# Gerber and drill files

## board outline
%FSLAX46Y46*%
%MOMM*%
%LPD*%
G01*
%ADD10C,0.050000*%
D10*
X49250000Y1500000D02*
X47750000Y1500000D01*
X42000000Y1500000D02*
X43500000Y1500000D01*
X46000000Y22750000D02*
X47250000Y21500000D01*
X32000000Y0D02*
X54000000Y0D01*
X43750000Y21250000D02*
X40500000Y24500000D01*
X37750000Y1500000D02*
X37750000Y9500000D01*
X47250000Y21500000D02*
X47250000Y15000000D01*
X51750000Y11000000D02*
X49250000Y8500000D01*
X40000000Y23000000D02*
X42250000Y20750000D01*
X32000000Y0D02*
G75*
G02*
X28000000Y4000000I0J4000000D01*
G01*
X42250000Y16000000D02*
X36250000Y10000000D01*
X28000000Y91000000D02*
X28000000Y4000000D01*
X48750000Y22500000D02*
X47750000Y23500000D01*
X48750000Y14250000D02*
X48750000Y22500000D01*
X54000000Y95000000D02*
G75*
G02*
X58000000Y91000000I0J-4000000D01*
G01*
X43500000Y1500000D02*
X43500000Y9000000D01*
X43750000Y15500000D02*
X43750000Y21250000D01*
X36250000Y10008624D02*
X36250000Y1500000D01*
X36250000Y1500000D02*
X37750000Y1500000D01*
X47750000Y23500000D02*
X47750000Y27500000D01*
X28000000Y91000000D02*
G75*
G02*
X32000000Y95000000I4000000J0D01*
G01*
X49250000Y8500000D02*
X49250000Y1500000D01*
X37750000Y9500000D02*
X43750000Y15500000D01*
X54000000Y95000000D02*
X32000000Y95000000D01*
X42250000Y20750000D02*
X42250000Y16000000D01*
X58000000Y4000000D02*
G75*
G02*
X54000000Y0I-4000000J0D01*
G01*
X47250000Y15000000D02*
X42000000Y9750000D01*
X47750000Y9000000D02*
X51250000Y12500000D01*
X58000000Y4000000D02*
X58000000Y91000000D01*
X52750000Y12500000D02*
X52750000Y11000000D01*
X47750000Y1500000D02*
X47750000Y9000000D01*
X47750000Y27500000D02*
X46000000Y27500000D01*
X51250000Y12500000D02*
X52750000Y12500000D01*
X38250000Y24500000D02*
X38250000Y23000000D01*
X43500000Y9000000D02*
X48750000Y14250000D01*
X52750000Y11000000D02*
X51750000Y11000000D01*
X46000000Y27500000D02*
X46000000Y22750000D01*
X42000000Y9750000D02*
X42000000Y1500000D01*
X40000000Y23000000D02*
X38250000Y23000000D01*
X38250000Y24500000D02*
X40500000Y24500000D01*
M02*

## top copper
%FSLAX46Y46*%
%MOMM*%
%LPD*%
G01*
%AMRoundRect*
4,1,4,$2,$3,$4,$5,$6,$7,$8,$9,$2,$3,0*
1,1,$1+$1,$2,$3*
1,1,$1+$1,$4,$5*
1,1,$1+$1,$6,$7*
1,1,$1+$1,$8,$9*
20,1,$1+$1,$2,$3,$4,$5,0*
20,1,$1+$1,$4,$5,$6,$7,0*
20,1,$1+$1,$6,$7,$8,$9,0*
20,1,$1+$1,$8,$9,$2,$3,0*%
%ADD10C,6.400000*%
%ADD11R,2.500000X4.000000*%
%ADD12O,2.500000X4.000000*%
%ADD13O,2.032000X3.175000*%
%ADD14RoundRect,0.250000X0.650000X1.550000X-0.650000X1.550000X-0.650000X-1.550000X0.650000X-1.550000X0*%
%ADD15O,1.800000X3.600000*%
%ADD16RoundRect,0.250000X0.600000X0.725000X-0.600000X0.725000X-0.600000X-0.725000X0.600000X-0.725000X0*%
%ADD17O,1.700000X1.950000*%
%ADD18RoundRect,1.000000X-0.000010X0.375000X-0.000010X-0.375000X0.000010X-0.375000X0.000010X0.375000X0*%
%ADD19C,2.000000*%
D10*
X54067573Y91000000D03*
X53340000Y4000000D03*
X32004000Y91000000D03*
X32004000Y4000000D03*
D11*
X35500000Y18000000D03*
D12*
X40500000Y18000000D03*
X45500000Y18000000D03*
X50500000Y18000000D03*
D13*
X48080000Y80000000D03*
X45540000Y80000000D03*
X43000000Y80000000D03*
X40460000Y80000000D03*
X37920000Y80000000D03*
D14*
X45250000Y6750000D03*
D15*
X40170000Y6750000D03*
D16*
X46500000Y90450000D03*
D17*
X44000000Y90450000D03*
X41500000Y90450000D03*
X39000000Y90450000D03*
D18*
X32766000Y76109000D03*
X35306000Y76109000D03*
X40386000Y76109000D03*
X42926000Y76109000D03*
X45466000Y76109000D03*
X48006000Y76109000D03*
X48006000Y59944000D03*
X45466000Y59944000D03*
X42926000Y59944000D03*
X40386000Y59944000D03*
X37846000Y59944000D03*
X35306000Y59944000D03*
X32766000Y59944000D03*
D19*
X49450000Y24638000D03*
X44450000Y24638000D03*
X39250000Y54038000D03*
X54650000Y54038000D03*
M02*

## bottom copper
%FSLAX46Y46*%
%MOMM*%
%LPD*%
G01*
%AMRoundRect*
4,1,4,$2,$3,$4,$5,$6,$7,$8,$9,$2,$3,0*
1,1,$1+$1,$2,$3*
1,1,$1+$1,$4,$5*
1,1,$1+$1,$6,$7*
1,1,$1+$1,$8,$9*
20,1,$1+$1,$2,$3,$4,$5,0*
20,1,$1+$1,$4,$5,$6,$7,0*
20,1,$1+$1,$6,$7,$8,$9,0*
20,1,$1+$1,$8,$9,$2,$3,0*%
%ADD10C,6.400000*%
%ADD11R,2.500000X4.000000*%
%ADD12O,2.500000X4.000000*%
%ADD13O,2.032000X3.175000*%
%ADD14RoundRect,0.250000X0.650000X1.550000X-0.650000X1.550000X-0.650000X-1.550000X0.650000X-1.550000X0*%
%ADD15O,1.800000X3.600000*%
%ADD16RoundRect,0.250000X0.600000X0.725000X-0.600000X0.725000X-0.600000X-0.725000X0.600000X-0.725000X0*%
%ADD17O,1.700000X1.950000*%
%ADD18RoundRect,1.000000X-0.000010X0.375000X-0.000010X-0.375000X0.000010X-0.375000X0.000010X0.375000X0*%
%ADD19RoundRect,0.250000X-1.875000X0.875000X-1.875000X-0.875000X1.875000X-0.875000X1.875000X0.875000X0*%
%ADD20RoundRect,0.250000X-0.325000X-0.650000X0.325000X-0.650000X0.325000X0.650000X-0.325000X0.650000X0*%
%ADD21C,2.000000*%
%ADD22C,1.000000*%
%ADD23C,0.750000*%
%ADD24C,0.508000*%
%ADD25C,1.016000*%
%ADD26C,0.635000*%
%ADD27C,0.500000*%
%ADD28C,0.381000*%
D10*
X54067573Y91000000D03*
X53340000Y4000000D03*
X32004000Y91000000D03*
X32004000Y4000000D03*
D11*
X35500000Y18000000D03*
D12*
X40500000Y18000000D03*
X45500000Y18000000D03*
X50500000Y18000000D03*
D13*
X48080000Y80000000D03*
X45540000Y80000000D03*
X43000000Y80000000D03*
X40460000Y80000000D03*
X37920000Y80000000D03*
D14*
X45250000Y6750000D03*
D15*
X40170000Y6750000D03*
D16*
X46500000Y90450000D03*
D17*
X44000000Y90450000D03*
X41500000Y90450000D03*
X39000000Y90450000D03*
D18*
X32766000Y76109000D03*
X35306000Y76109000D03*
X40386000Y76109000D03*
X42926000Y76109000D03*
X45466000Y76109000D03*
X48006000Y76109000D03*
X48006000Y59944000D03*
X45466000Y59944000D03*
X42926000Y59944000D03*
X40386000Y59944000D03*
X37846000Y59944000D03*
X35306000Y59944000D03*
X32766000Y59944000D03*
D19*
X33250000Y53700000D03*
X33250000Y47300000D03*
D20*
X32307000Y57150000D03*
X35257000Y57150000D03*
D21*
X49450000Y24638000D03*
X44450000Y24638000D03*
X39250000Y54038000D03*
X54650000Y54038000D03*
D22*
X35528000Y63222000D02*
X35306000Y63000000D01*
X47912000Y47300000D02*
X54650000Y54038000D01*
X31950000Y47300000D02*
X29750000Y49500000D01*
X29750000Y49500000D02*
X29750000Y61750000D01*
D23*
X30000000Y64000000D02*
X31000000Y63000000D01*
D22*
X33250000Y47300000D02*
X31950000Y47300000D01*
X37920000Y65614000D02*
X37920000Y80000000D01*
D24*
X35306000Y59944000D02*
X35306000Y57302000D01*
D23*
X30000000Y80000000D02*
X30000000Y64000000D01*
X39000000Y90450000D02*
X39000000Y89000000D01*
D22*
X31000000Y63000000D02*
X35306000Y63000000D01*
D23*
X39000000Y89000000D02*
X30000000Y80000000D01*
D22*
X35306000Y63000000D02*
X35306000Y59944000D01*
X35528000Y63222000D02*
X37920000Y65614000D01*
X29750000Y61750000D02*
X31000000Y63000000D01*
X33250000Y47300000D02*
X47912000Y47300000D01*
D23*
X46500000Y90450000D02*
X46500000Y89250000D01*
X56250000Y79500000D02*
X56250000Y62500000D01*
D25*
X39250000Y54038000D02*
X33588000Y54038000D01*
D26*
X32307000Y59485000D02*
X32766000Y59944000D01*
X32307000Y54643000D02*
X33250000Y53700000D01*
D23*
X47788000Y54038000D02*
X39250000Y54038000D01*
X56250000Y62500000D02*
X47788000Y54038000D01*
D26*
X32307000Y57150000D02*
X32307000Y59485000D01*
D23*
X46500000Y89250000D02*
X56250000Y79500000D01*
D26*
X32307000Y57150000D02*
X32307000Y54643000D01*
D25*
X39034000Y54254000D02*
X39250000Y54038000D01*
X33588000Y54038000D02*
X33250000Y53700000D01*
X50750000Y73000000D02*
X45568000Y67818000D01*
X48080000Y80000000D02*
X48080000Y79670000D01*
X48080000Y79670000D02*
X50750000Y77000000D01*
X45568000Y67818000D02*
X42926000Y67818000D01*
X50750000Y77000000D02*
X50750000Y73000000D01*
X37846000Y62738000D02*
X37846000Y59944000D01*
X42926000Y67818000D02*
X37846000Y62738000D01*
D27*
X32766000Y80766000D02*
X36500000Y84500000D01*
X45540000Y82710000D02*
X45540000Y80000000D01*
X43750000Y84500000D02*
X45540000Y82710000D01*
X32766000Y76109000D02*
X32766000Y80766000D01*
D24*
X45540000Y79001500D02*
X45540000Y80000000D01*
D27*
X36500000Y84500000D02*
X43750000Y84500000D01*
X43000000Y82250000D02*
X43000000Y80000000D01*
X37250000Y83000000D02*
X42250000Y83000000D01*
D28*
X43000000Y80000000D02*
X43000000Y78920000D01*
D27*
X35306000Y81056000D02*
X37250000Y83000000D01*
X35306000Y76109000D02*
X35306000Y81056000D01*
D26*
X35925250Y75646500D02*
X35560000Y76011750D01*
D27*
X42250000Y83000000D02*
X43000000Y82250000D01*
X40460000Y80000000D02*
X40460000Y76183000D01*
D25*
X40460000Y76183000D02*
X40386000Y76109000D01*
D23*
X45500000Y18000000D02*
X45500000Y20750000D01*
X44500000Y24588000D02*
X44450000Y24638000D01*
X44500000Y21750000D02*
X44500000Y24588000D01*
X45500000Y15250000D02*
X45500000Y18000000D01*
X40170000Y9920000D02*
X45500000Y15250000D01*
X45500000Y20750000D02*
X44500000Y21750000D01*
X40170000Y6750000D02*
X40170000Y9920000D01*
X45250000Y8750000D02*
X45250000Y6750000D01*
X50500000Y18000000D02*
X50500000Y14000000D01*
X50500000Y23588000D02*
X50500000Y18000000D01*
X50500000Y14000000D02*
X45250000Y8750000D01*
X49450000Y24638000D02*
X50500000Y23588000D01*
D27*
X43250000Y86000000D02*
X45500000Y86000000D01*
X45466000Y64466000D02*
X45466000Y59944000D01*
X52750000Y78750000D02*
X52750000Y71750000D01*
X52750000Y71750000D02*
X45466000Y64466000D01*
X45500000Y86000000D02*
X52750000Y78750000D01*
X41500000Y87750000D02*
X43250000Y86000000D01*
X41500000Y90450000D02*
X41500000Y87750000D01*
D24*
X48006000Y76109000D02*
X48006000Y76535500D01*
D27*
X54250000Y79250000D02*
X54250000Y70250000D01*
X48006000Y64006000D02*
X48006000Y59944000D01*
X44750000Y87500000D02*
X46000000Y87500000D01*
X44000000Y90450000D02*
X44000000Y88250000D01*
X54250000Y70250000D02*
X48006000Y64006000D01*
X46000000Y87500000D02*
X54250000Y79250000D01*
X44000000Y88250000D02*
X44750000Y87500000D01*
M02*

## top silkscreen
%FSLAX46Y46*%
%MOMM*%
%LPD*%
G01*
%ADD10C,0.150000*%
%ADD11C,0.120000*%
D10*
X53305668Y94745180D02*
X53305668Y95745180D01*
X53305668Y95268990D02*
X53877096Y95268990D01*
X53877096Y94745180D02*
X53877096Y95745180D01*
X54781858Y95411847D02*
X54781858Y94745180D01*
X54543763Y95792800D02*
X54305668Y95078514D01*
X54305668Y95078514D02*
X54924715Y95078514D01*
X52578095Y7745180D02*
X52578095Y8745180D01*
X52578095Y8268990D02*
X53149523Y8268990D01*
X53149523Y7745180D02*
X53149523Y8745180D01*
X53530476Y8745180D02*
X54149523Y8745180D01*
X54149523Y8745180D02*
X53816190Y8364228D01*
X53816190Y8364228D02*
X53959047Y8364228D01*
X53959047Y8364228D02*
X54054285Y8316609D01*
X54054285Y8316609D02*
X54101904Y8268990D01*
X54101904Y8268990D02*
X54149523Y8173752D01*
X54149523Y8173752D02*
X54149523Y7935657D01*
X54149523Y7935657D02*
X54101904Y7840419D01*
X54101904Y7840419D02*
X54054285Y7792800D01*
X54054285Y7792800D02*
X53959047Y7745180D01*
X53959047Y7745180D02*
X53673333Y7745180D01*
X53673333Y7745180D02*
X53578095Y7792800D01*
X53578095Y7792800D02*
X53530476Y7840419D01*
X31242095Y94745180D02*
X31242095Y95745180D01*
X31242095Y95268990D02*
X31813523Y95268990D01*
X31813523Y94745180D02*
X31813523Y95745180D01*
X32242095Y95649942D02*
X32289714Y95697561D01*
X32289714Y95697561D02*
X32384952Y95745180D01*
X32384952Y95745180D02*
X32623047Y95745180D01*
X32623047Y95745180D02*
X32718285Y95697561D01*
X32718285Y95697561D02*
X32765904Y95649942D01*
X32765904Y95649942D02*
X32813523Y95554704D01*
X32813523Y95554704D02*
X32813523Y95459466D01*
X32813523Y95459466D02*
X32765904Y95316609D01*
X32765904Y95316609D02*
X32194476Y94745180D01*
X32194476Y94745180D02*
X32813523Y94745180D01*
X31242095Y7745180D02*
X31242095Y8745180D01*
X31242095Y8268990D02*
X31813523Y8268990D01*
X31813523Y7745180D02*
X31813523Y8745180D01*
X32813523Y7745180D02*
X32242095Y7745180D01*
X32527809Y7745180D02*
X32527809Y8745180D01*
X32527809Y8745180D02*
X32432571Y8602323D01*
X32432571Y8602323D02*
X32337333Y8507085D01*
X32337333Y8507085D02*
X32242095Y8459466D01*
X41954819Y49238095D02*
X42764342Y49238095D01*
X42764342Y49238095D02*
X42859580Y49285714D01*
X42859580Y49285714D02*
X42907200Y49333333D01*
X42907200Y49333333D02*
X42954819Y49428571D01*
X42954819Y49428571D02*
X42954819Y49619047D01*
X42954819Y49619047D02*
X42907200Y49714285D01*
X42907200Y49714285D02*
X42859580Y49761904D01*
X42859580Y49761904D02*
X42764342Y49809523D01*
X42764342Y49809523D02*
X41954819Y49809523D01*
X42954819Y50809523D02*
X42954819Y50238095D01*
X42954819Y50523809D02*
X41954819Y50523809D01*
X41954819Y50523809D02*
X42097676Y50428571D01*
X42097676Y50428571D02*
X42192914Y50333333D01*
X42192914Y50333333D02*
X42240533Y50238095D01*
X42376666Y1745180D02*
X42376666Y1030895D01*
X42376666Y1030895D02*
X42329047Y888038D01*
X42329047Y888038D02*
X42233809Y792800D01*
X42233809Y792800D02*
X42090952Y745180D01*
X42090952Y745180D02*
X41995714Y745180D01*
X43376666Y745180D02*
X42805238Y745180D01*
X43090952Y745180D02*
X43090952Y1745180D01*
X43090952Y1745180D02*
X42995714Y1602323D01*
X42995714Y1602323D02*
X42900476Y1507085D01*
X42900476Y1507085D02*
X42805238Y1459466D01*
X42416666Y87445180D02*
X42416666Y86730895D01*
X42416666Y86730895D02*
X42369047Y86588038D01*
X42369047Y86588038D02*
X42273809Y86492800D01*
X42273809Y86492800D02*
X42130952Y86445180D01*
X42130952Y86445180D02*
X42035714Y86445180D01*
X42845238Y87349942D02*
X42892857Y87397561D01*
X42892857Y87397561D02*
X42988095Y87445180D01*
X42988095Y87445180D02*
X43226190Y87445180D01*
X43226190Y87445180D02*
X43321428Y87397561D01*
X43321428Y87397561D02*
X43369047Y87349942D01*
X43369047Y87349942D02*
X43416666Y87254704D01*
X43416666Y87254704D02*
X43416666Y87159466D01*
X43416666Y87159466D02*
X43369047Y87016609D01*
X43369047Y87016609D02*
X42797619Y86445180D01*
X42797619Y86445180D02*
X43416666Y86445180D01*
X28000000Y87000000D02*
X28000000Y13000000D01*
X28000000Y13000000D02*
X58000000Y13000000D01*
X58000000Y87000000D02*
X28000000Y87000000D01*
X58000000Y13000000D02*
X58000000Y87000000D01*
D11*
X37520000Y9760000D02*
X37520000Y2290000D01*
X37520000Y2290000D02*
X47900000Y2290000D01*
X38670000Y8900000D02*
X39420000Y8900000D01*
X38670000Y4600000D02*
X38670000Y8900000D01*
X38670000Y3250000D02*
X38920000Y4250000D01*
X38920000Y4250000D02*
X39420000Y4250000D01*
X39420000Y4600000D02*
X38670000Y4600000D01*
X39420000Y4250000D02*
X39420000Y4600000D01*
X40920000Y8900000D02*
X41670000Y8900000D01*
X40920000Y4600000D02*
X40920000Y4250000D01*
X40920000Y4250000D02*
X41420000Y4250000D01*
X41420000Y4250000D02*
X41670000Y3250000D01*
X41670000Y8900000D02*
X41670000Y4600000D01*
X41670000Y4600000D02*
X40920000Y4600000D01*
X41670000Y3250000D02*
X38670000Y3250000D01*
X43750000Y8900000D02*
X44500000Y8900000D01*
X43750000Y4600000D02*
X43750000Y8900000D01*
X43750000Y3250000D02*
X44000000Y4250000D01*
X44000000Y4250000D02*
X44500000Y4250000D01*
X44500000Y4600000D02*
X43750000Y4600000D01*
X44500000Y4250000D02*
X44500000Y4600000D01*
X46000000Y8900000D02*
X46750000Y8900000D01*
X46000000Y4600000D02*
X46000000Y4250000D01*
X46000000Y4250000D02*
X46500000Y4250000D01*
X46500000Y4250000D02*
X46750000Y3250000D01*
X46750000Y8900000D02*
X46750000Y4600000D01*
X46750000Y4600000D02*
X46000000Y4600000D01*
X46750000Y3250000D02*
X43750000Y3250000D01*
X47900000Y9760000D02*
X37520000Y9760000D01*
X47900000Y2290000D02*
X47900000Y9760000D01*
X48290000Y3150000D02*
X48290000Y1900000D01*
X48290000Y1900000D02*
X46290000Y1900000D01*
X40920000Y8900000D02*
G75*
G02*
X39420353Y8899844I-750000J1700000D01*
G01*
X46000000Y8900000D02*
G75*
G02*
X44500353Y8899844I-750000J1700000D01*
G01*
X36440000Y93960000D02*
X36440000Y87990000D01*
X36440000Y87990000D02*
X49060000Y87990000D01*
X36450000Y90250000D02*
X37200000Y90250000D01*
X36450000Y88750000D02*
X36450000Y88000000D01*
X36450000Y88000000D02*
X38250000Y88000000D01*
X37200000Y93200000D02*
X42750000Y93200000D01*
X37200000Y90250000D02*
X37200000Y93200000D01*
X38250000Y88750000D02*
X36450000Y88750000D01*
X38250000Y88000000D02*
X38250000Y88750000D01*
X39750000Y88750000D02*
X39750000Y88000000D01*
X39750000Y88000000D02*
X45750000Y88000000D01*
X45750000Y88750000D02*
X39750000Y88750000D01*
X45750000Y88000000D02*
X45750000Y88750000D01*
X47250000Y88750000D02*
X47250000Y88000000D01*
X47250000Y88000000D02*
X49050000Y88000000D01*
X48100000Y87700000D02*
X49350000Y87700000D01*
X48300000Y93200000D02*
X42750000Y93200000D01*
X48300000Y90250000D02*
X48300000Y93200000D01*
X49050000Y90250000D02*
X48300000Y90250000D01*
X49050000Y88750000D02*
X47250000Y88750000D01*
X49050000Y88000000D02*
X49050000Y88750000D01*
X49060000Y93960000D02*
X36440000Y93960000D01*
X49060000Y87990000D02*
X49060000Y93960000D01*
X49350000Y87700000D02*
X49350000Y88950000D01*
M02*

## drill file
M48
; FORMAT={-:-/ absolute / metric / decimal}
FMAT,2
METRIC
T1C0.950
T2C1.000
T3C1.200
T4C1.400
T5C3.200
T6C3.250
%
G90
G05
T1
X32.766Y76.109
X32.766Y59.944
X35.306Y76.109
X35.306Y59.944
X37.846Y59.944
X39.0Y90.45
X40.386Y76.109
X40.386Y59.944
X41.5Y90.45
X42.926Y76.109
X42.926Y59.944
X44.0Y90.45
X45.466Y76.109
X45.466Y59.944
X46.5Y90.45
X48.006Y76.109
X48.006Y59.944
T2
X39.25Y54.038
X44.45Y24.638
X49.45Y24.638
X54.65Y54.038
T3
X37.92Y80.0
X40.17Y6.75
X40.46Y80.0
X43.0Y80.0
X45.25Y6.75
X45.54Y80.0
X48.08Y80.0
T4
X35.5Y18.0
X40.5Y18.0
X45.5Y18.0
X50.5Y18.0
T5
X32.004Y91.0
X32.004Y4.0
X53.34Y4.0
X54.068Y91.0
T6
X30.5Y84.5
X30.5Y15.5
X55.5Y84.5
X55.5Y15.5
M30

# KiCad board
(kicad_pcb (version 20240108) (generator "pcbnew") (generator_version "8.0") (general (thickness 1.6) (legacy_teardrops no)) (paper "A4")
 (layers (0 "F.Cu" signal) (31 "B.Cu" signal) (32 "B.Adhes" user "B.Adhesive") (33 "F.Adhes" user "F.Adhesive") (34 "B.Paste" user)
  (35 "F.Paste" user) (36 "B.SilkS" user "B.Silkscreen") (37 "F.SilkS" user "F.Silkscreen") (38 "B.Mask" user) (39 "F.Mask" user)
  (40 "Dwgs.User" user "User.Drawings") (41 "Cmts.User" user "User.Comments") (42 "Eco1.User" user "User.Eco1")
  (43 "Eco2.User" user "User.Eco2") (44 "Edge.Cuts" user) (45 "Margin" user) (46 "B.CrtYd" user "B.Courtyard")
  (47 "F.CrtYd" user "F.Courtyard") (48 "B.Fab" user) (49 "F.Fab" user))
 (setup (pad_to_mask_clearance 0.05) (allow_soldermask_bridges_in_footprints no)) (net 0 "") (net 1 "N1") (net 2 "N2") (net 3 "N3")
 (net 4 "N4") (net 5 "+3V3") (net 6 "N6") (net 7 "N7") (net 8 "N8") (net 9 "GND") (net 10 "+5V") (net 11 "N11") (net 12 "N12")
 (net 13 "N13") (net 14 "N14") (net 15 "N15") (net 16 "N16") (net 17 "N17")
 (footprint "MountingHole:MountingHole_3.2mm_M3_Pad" (layer "F.Cu") (at 54.067573 -91)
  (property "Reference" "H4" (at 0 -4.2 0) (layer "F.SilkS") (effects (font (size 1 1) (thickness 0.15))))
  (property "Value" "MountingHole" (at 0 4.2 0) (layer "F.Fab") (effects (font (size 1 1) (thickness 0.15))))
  (pad "1" thru_hole circle (at 0 0) (size 6.4 6.4) (drill 3.2) (layers "*.Cu" "*.Mask") (remove_unused_layers no)))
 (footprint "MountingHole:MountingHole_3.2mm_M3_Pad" (layer "F.Cu") (at 53.34 -4)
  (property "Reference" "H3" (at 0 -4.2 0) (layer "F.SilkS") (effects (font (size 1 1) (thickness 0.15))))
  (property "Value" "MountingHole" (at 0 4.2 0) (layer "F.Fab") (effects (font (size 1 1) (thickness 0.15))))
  (pad "1" thru_hole circle (at 0 0) (size 6.4 6.4) (drill 3.2) (layers "*.Cu" "*.Mask") (remove_unused_layers no)))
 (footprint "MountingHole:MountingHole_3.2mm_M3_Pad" (layer "F.Cu") (at 32.004 -91)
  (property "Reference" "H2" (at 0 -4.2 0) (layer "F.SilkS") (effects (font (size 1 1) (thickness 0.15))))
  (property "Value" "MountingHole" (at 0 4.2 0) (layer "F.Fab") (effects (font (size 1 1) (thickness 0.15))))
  (pad "1" thru_hole circle (at 0 0) (size 6.4 6.4) (drill 3.2) (layers "*.Cu" "*.Mask") (remove_unused_layers no)))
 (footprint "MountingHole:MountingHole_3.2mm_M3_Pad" (layer "F.Cu") (at 32.004 -4)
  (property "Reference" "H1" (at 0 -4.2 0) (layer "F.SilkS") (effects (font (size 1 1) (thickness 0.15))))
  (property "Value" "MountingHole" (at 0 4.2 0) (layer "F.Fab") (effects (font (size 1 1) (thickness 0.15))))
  (pad "1" thru_hole circle (at 0 0) (size 6.4 6.4) (drill 3.2) (layers "*.Cu" "*.Mask") (remove_unused_layers no)))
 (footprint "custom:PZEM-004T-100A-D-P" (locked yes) (layer "F.Cu") (at 43 -50 90)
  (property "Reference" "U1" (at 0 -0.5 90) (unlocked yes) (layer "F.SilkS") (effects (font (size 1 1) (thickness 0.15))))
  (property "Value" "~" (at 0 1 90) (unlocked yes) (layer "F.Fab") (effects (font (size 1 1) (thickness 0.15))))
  (fp_line (start 37 -15) (end -37 -15) (stroke (width 0.15) (type default)) (layer "F.SilkS"))
  (fp_line (start -37 -15) (end -37 15) (stroke (width 0.15) (type default)) (layer "F.SilkS"))
  (fp_line (start 37 15) (end 37 -15) (stroke (width 0.15) (type default)) (layer "F.SilkS"))
  (fp_line (start -37 15) (end 37 15) (stroke (width 0.15) (type default)) (layer "F.SilkS"))
  (pad "" np_thru_hole circle (at -34.5 -12.5 90) (size 3.25 3.25) (drill 3.25) (layers "F&B.Cu" "*.Mask"))
  (pad "" np_thru_hole circle (at -34.5 12.5 180) (size 3.25 3.25) (drill 3.25) (layers "F&B.Cu" "*.Mask"))
  (pad "" np_thru_hole circle (at 34.5 -12.5 90) (size 3.25 3.25) (drill 3.25) (layers "F&B.Cu" "*.Mask"))
  (pad "" np_thru_hole circle (at 34.5 12.5 90) (size 3.25 3.25) (drill 3.25) (layers "F&B.Cu" "*.Mask"))
  (pad "1" thru_hole rect (at -32 -7.5 90) (size 4 2.5) (drill 1.4) (layers "*.Cu" "*.Mask") (remove_unused_layers no) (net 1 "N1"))
  (pad "2" thru_hole oval (at -32 -2.5 90) (size 4 2.5) (drill 1.4) (layers "*.Cu" "*.Mask") (remove_unused_layers no) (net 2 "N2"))
  (pad "3" thru_hole oval (at -32 2.5 90) (size 4 2.5) (drill 1.4) (layers "*.Cu" "*.Mask") (remove_unused_layers no) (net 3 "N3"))
  (pad "4" thru_hole oval (at -32 7.5 90) (size 4 2.5) (drill 1.4) (layers "*.Cu" "*.Mask") (remove_unused_layers no) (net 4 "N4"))
  (pad "5" thru_hole oval (at 30 5.08 90) (size 3.175 2.032) (drill 1.2) (layers "*.Cu" "*.Mask") (remove_unused_layers no) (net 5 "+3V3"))
  (pad "6" thru_hole oval (at 30 2.54 90) (size 3.175 2.032) (drill 1.2) (layers "*.Cu" "*.Mask") (remove_unused_layers no) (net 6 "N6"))
  (pad "7" thru_hole oval (at 30 0 90) (size 3.175 2.032) (drill 1.2) (layers "*.Cu" "*.Mask") (remove_unused_layers no) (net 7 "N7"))
  (pad "8" thru_hole oval (at 30 -2.54 90) (size 3.175 2.032) (drill 1.2) (layers "*.Cu" "*.Mask") (remove_unused_layers no) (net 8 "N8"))
  (pad "9" thru_hole oval (at 30 -5.08 90) (size 3.175 2.032) (drill 1.2) (layers "*.Cu" "*.Mask") (remove_unused_layers no) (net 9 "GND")))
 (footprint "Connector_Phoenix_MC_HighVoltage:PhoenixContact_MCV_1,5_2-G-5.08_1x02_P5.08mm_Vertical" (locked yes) (layer "F.Cu")
  (at 45.25 -6.75 180)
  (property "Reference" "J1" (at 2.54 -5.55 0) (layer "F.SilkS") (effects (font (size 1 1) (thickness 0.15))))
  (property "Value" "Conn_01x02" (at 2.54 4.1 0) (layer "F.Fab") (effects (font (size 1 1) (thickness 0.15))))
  (fp_line (start 7.73 3.01) (end 7.73 -4.46) (stroke (width 0.12) (type solid)) (layer "F.SilkS"))
  (fp_line (start 7.73 -4.46) (end -2.65 -4.46) (stroke (width 0.12) (type solid)) (layer "F.SilkS"))
  (fp_line (start 6.58 2.15) (end 5.83 2.15) (stroke (width 0.12) (type solid)) (layer "F.SilkS"))
  (fp_line (start 6.58 -2.15) (end 6.58 2.15) (stroke (width 0.12) (type solid)) (layer "F.SilkS"))
  (fp_line (start 6.58 -3.5) (end 6.33 -2.5) (stroke (width 0.12) (type solid)) (layer "F.SilkS"))
  (fp_line (start 6.33 -2.5) (end 5.83 -2.5) (stroke (width 0.12) (type solid)) (layer "F.SilkS"))
  (fp_line (start 5.83 -2.15) (end 6.58 -2.15) (stroke (width 0.12) (type solid)) (layer "F.SilkS"))
  (fp_line (start 5.83 -2.5) (end 5.83 -2.15) (stroke (width 0.12) (type solid)) (layer "F.SilkS"))
  (fp_line (start 4.33 2.15) (end 3.58 2.15) (stroke (width 0.12) (type solid)) (layer "F.SilkS"))
  (fp_line (start 4.33 -2.15) (end 4.33 -2.5) (stroke (width 0.12) (type solid)) (layer "F.SilkS"))
  (fp_line (start 4.33 -2.5) (end 3.83 -2.5) (stroke (width 0.12) (type solid)) (layer "F.SilkS"))
  (fp_line (start 3.83 -2.5) (end 3.58 -3.5) (stroke (width 0.12) (type solid)) (layer "F.SilkS"))
  (fp_line (start 3.58 2.15) (end 3.58 -2.15) (stroke (width 0.12) (type solid)) (layer "F.SilkS"))
  (fp_line (start 3.58 -2.15) (end 4.33 -2.15) (stroke (width 0.12) (type solid)) (layer "F.SilkS"))
  (fp_line (start 3.58 -3.5) (end 6.58 -3.5) (stroke (width 0.12) (type solid)) (layer "F.SilkS"))
  (fp_line (start 1.5 2.15) (end 0.75 2.15) (stroke (width 0.12) (type solid)) (layer "F.SilkS"))
  (fp_line (start 1.5 -2.15) (end 1.5 2.15) (stroke (width 0.12) (type solid)) (layer "F.SilkS"))
  (fp_line (start 1.5 -3.5) (end 1.25 -2.5) (stroke (width 0.12) (type solid)) (layer "F.SilkS"))
  (fp_line (start 1.25 -2.5) (end 0.75 -2.5) (stroke (width 0.12) (type solid)) (layer "F.SilkS"))
  (fp_line (start 0.75 -2.15) (end 1.5 -2.15) (stroke (width 0.12) (type solid)) (layer "F.SilkS"))
  (fp_line (start 0.75 -2.5) (end 0.75 -2.15) (stroke (width 0.12) (type solid)) (layer "F.SilkS"))
  (fp_line (start -0.75 2.15) (end -1.5 2.15) (stroke (width 0.12) (type solid)) (layer "F.SilkS"))
  (fp_line (start -0.75 -2.15) (end -0.75 -2.5) (stroke (width 0.12) (type solid)) (layer "F.SilkS"))
  (fp_line (start -0.75 -2.5) (end -1.25 -2.5) (stroke (width 0.12) (type solid)) (layer "F.SilkS"))
  (fp_line (start -1.25 -2.5) (end -1.5 -3.5) (stroke (width 0.12) (type solid)) (layer "F.SilkS"))
  (fp_line (start -1.5 2.15) (end -1.5 -2.15) (stroke (width 0.12) (type solid)) (layer "F.SilkS"))
  (fp_line (start -1.5 -2.15) (end -0.75 -2.15) (stroke (width 0.12) (type solid)) (layer "F.SilkS"))
  (fp_line (start -1.5 -3.5) (end 1.5 -3.5) (stroke (width 0.12) (type solid)) (layer "F.SilkS"))
  (fp_line (start -2.65 3.01) (end 7.73 3.01) (stroke (width 0.12) (type solid)) (layer "F.SilkS"))
  (fp_line (start -2.65 -4.46) (end -2.65 3.01) (stroke (width 0.12) (type solid)) (layer "F.SilkS"))
  (fp_line (start -3.04 -3.6) (end -3.04 -4.85) (stroke (width 0.12) (type solid)) (layer "F.SilkS"))
  (fp_line (start -3.04 -4.85) (end -1.04 -4.85) (stroke (width 0.12) (type solid)) (layer "F.SilkS"))
  (fp_arc (start 4.33 2.15) (mid 5.079807 1.99191) (end 5.829647 2.149844) (stroke (width 0.12) (type solid)) (layer "F.SilkS"))
  (fp_arc (start -0.75 2.15) (mid -0.000193 1.99191) (end 0.749647 2.149844) (stroke (width 0.12) (type solid)) (layer "F.SilkS"))
  (pad "1" thru_hole roundrect (at 0 0 180) (size 1.8 3.6) (drill 1.2) (layers "*.Cu" "*.Mask") (remove_unused_layers no)
   (roundrect_rratio 0.138889) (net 4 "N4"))
  (pad "2" thru_hole oval (at 5.08 0 180) (size 1.8 3.6) (drill 1.2) (layers "*.Cu" "*.Mask") (remove_unused_layers no) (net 3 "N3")))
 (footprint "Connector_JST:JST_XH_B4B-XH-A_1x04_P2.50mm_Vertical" (layer "F.Cu") (at 46.5 -90.45 180)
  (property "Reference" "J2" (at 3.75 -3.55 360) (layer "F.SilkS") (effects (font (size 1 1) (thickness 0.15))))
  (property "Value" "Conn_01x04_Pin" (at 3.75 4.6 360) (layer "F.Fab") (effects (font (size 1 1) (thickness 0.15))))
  (fp_line (start 10.06 3.51) (end 10.06 -2.46) (stroke (width 0.12) (type solid)) (layer "F.SilkS"))
  (fp_line (start 10.06 -2.46) (end -2.56 -2.46) (stroke (width 0.12) (type solid)) (layer "F.SilkS"))
  (fp_line (start 10.05 -0.2) (end 9.3 -0.2) (stroke (width 0.12) (type solid)) (layer "F.SilkS"))
  (fp_line (start 10.05 -1.7) (end 10.05 -2.45) (stroke (width 0.12) (type solid)) (layer "F.SilkS"))
  (fp_line (start 10.05 -2.45) (end 8.25 -2.45) (stroke (width 0.12) (type solid)) (layer "F.SilkS"))
  (fp_line (start 9.3 2.75) (end 3.75 2.75) (stroke (width 0.12) (type solid)) (layer "F.SilkS"))
  (fp_line (start 9.3 -0.2) (end 9.3 2.75) (stroke (width 0.12) (type solid)) (layer "F.SilkS"))
  (fp_line (start 8.25 -1.7) (end 10.05 -1.7) (stroke (width 0.12) (type solid)) (layer "F.SilkS"))
  (fp_line (start 8.25 -2.45) (end 8.25 -1.7) (stroke (width 0.12) (type solid)) (layer "F.SilkS"))
  (fp_line (start 6.75 -1.7) (end 6.75 -2.45) (stroke (width 0.12) (type solid)) (layer "F.SilkS"))
  (fp_line (start 6.75 -2.45) (end 0.75 -2.45) (stroke (width 0.12) (type solid)) (layer "F.SilkS"))
  (fp_line (start 0.75 -1.7) (end 6.75 -1.7) (stroke (width 0.12) (type solid)) (layer "F.SilkS"))
  (fp_line (start 0.75 -2.45) (end 0.75 -1.7) (stroke (width 0.12) (type solid)) (layer "F.SilkS"))
  (fp_line (start -0.75 -1.7) (end -0.75 -2.45) (stroke (width 0.12) (type solid)) (layer "F.SilkS"))
  (fp_line (start -0.75 -2.45) (end -2.55 -2.45) (stroke (width 0.12) (type solid)) (layer "F.SilkS"))
  (fp_line (start -1.6 -2.75) (end -2.85 -2.75) (stroke (width 0.12) (type solid)) (layer "F.SilkS"))
  (fp_line (start -1.8 2.75) (end 3.75 2.75) (stroke (width 0.12) (type solid)) (layer "F.SilkS"))
  (fp_line (start -1.8 -0.2) (end -1.8 2.75) (stroke (width 0.12) (type solid)) (layer "F.SilkS"))
  (fp_line (start -2.55 -0.2) (end -1.8 -0.2) (stroke (width 0.12) (type solid)) (layer "F.SilkS"))
  (fp_line (start -2.55 -1.7) (end -0.75 -1.7) (stroke (width 0.12) (type solid)) (layer "F.SilkS"))
  (fp_line (start -2.55 -2.45) (end -2.55 -1.7) (stroke (width 0.12) (type solid)) (layer "F.SilkS"))
  (fp_line (start -2.56 3.51) (end 10.06 3.51) (stroke (width 0.12) (type solid)) (layer "F.SilkS"))
  (fp_line (start -2.56 -2.46) (end -2.56 3.51) (stroke (width 0.12) (type solid)) (layer "F.SilkS"))
  (fp_line (start -2.85 -2.75) (end -2.85 -1.5) (stroke (width 0.12) (type solid)) (layer "F.SilkS"))
  (pad "1" thru_hole roundrect (at 0 0 180) (size 1.7 1.95) (drill 0.95) (layers "*.Cu" "*.Mask") (remove_unused_layers no)
   (roundrect_rratio 0.147059) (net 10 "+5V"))
  (pad "2" thru_hole oval (at 2.5 0 180) (size 1.7 1.95) (drill 0.95) (layers "*.Cu" "*.Mask") (remove_unused_layers no) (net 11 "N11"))
  (pad "3" thru_hole oval (at 5 0 180) (size 1.7 1.95) (drill 0.95) (layers "*.Cu" "*.Mask") (remove_unused_layers no) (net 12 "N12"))
  (pad "4" thru_hole oval (at 7.5 0 180) (size 1.7 1.95) (drill 0.95) (layers "*.Cu" "*.Mask") (remove_unused_layers no) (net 9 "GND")))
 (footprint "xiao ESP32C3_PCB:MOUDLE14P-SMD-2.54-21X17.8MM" (layer "B.Cu") (at 50.886 -76.944 -90)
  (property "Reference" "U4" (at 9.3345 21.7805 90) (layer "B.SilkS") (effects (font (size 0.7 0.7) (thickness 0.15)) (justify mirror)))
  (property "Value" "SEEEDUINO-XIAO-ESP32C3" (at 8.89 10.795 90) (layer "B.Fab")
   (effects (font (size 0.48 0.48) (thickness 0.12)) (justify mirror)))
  (pad "1" thru_hole roundrect (at 0.835 18.12 270) (size 2.75 2) (drill 0.95) (layers "*.Cu" "*.Mask") (remove_unused_layers no)
   (roundrect_rratio 0.5) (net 6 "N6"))
  (pad "2" thru_hole roundrect (at 0.835 15.58 270) (size 2.75 2) (drill 0.95) (layers "*.Cu" "*.Mask") (remove_unused_layers no)
   (roundrect_rratio 0.5) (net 7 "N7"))
  (pad "4" thru_hole roundrect (at 0.835 10.5 270) (size 2.75 2) (drill 0.95) (layers "*.Cu" "*.Mask") (remove_unused_layers no)
   (roundrect_rratio 0.5) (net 8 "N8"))
  (pad "5" thru_hole roundrect (at 0.835 7.96 270) (size 2.75 2) (drill 0.95) (layers "*.Cu" "*.Mask") (remove_unused_layers no)
   (roundrect_rratio 0.5) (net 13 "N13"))
  (pad "6" thru_hole roundrect (at 0.835 5.42 270) (size 2.75 2) (drill 0.95) (layers "*.Cu" "*.Mask") (remove_unused_layers no)
   (roundrect_rratio 0.5) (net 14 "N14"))
  (pad "7" thru_hole roundrect (at 0.835 2.88 270) (size 2.75 2) (drill 0.95) (layers "*.Cu" "*.Mask") (remove_unused_layers no)
   (roundrect_rratio 0.5) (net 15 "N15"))
  (pad "8" thru_hole roundrect (at 17 2.88 270) (size 2.75 2) (drill 0.95) (layers "*.Cu" "*.Mask") (remove_unused_layers no)
   (roundrect_rratio 0.5) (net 11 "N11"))
  (pad "9" thru_hole roundrect (at 17 5.42 270) (size 2.75 2) (drill 0.95) (layers "*.Cu" "*.Mask") (remove_unused_layers no)
   (roundrect_rratio 0.5) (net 12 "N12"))
  (pad "10" thru_hole roundrect (at 17 7.96 270) (size 2.75 2) (drill 0.95) (layers "*.Cu" "*.Mask") (remove_unused_layers no)
   (roundrect_rratio 0.5) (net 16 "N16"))
  (pad "11" thru_hole roundrect (at 17 10.5 270) (size 2.75 2) (drill 0.95) (layers "*.Cu" "*.Mask") (remove_unused_layers no)
   (roundrect_rratio 0.5) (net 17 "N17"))
  (pad "12" thru_hole roundrect (at 17 13.04 270) (size 2.75 2) (drill 0.95) (layers "*.Cu" "*.Mask") (remove_unused_layers no)
   (roundrect_rratio 0.5) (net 5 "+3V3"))
  (pad "13" thru_hole roundrect (at 17 15.58 270) (size 2.75 2) (drill 0.95) (layers "*.Cu" "*.Mask") (remove_unused_layers no)
   (roundrect_rratio 0.5) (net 9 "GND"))
  (pad "14" thru_hole roundrect (at 17 18.12 270) (size 2.75 2) (drill 0.95) (layers "*.Cu" "*.Mask") (remove_unused_layers no)
   (roundrect_rratio 0.5) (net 10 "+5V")))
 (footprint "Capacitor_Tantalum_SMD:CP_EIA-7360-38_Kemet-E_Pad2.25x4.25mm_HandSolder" (layer "B.Cu") (at 33.25 -50.5 -90)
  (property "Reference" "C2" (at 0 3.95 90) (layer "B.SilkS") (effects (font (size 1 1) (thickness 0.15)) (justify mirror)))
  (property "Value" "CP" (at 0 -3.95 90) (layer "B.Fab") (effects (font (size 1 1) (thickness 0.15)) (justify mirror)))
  (pad "1" smd roundrect (at -3.2 0 270) (size 2.25 4.25) (layers "B.Cu" "B.Paste" "B.Mask") (roundrect_rratio 0.111111) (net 10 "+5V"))
  (pad "2" smd roundrect (at 3.2 0 270) (size 2.25 4.25) (layers "B.Cu" "B.Paste" "B.Mask") (roundrect_rratio 0.111111) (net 9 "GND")))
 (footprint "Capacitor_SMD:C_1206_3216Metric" (layer "B.Cu") (at 33.782 -57.15)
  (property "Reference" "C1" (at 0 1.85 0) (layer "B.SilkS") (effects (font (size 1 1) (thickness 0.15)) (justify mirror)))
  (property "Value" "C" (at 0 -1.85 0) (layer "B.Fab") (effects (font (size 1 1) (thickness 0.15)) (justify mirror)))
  (pad "1" smd roundrect (at -1.475 0) (size 1.15 1.8) (layers "B.Cu" "B.Paste" "B.Mask") (roundrect_rratio 0.217391) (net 10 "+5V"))
  (pad "2" smd roundrect (at 1.475 0) (size 1.15 1.8) (layers "B.Cu" "B.Paste" "B.Mask") (roundrect_rratio 0.217391) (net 9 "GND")))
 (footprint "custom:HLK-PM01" (layer "B.Cu") (at 46.95 -24.638 90)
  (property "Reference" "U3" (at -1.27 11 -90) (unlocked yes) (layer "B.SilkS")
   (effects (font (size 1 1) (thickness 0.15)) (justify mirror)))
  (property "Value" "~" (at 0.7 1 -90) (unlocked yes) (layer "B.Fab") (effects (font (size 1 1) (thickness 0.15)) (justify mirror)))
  (pad "1" thru_hole circle (at 0 2.5 90) (size 2 2) (drill 1) (layers "*.Cu" "*.Mask") (remove_unused_layers no) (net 4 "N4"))
  (pad "2" thru_hole circle (at 0 -2.5 90) (size 2 2) (drill 1) (layers "*.Cu" "*.Mask") (remove_unused_layers no) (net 3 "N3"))
  (pad "3" thru_hole circle (at 29.4 -7.7 90) (size 2 2) (drill 1) (layers "*.Cu" "*.Mask") (remove_unused_layers no) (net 10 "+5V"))
  (pad "4" thru_hole circle (at 29.4 7.7 90) (size 2 2) (drill 1) (layers "*.Cu" "*.Mask") (remove_unused_layers no) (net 9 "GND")))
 (gr_line (start 49.25 -1.5) (end 47.75 -1.5) (stroke (width 0.05) (type default)) (layer "Edge.Cuts"))
 (gr_line (start 42 -1.5) (end 43.5 -1.5) (stroke (width 0.05) (type default)) (layer "Edge.Cuts"))
 (gr_line (start 46 -22.75) (end 47.25 -21.5) (stroke (width 0.05) (type default)) (layer "Edge.Cuts"))
 (gr_line (start 32 0) (end 54 0) (stroke (width 0.05) (type solid)) (layer "Edge.Cuts"))
 (gr_line (start 43.75 -21.25) (end 40.5 -24.5) (stroke (width 0.05) (type default)) (layer "Edge.Cuts"))
 (gr_line (start 37.75 -1.5) (end 37.75 -9.5) (stroke (width 0.05) (type default)) (layer "Edge.Cuts"))
 (gr_line (start 47.25 -21.5) (end 47.25 -15) (stroke (width 0.05) (type default)) (layer "Edge.Cuts"))
 (gr_line (start 51.75 -11) (end 49.25 -8.5) (stroke (width 0.05) (type default)) (layer "Edge.Cuts"))
 (gr_line (start 40 -23) (end 42.25 -20.75) (stroke (width 0.05) (type default)) (layer "Edge.Cuts"))
 (gr_arc (start 32 0) (mid 29.171573 -1.171573) (end 28 -4) (stroke (width 0.05) (type default)) (layer "Edge.Cuts"))
 (gr_line (start 42.25 -16) (end 36.25 -10) (stroke (width 0.05) (type default)) (layer "Edge.Cuts"))
 (gr_line (start 28 -91) (end 28 -4) (stroke (width 0.05) (type solid)) (layer "Edge.Cuts"))
 (gr_line (start 48.75 -22.5) (end 47.75 -23.5) (stroke (width 0.05) (type default)) (layer "Edge.Cuts"))
 (gr_line (start 48.75 -14.25) (end 48.75 -22.5) (stroke (width 0.05) (type default)) (layer "Edge.Cuts"))
 (gr_arc (start 54 -95) (mid 56.828427 -93.828427) (end 58 -91) (stroke (width 0.05) (type default)) (layer "Edge.Cuts"))
 (gr_line (start 43.5 -1.5) (end 43.5 -9) (stroke (width 0.05) (type default)) (layer "Edge.Cuts"))
 (gr_line (start 43.75 -15.5) (end 43.75 -21.25) (stroke (width 0.05) (type default)) (layer "Edge.Cuts"))
 (gr_line (start 36.25 -10.008624) (end 36.25 -1.5) (stroke (width 0.05) (type default)) (layer "Edge.Cuts"))
 (gr_line (start 36.25 -1.5) (end 37.75 -1.5) (stroke (width 0.05) (type default)) (layer "Edge.Cuts"))
 (gr_line (start 47.75 -23.5) (end 47.75 -27.5) (stroke (width 0.05) (type default)) (layer "Edge.Cuts"))
 (gr_arc (start 28 -91) (mid 29.171573 -93.828427) (end 32 -95) (stroke (width 0.05) (type default)) (layer "Edge.Cuts"))
 (gr_line (start 49.25 -8.5) (end 49.25 -1.5) (stroke (width 0.05) (type default)) (layer "Edge.Cuts"))
 (gr_line (start 37.75 -9.5) (end 43.75 -15.5) (stroke (width 0.05) (type default)) (layer "Edge.Cuts"))
 (gr_line (start 54 -95) (end 32 -95) (stroke (width 0.05) (type solid)) (layer "Edge.Cuts"))
 (gr_line (start 42.25 -20.75) (end 42.25 -16) (stroke (width 0.05) (type default)) (layer "Edge.Cuts"))
 (gr_arc (start 58 -4) (mid 56.828427 -1.171573) (end 54 0) (stroke (width 0.05) (type default)) (layer "Edge.Cuts"))
 (gr_line (start 47.25 -15) (end 42 -9.75) (stroke (width 0.05) (type default)) (layer "Edge.Cuts"))
 (gr_line (start 47.75 -9) (end 51.25 -12.5) (stroke (width 0.05) (type default)) (layer "Edge.Cuts"))
 (gr_line (start 58 -4) (end 58 -91) (stroke (width 0.05) (type solid)) (layer "Edge.Cuts"))
 (gr_line (start 52.75 -12.5) (end 52.75 -11) (stroke (width 0.05) (type default)) (layer "Edge.Cuts"))
 (gr_line (start 47.75 -1.5) (end 47.75 -9) (stroke (width 0.05) (type default)) (layer "Edge.Cuts"))
 (gr_line (start 47.75 -27.5) (end 46 -27.5) (stroke (width 0.05) (type default)) (layer "Edge.Cuts"))
 (gr_line (start 51.25 -12.5) (end 52.75 -12.5) (stroke (width 0.05) (type default)) (layer "Edge.Cuts"))
 (gr_line (start 38.25 -24.5) (end 38.25 -23) (stroke (width 0.05) (type default)) (layer "Edge.Cuts"))
 (gr_line (start 43.5 -9) (end 48.75 -14.25) (stroke (width 0.05) (type default)) (layer "Edge.Cuts"))
 (gr_line (start 52.75 -11) (end 51.75 -11) (stroke (width 0.05) (type default)) (layer "Edge.Cuts"))
 (gr_line (start 46 -27.5) (end 46 -22.75) (stroke (width 0.05) (type default)) (layer "Edge.Cuts"))
 (gr_line (start 42 -9.75) (end 42 -1.5) (stroke (width 0.05) (type default)) (layer "Edge.Cuts"))
 (gr_line (start 40 -23) (end 38.25 -23) (stroke (width 0.05) (type default)) (layer "Edge.Cuts"))
 (gr_line (start 38.25 -24.5) (end 40.5 -24.5) (stroke (width 0.05) (type default)) (layer "Edge.Cuts"))
 (segment (start 35.528 -63.222) (end 35.306 -63) (width 1) (layer "B.Cu") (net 9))
 (segment (start 47.912 -47.3) (end 54.65 -54.038) (width 1) (layer "B.Cu") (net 9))
 (segment (start 31.95 -47.3) (end 29.75 -49.5) (width 1) (layer "B.Cu") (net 9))
 (segment (start 29.75 -49.5) (end 29.75 -61.75) (width 1) (layer "B.Cu") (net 9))
 (segment (start 30 -64) (end 31 -63) (width 0.75) (layer "B.Cu") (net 9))
 (segment (start 33.25 -47.3) (end 31.95 -47.3) (width 1) (layer "B.Cu") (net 9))
 (segment (start 37.92 -65.614) (end 37.92 -80) (width 1) (layer "B.Cu") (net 9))
 (segment (start 35.306 -59.944) (end 35.306 -57.302) (width 0.508) (layer "B.Cu") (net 9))
 (segment (start 30 -80) (end 30 -64) (width 0.75) (layer "B.Cu") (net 9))
 (segment (start 39 -90.45) (end 39 -89) (width 0.75) (layer "B.Cu") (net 9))
 (segment (start 31 -63) (end 35.306 -63) (width 1) (layer "B.Cu") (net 9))
 (segment (start 39 -89) (end 30 -80) (width 0.75) (layer "B.Cu") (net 9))
 (segment (start 35.306 -63) (end 35.306 -59.944) (width 1) (layer "B.Cu") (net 9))
 (segment (start 35.528 -63.222) (end 37.92 -65.614) (width 1) (layer "B.Cu") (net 9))
 (segment (start 29.75 -61.75) (end 31 -63) (width 1) (layer "B.Cu") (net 9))
 (segment (start 33.25 -47.3) (end 47.912 -47.3) (width 1) (layer "B.Cu") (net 9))
 (segment (start 46.5 -90.45) (end 46.5 -89.25) (width 0.75) (layer "B.Cu") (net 10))
 (segment (start 56.25 -79.5) (end 56.25 -62.5) (width 0.75) (layer "B.Cu") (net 10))
 (segment (start 39.25 -54.038) (end 33.588 -54.038) (width 1.016) (layer "B.Cu") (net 10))
 (segment (start 32.307 -59.485) (end 32.766 -59.944) (width 0.635) (layer "B.Cu") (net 10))
 (segment (start 32.307 -54.643) (end 33.25 -53.7) (width 0.635) (layer "B.Cu") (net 10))
 (segment (start 47.788 -54.038) (end 39.25 -54.038) (width 0.75) (layer "B.Cu") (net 10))
 (segment (start 56.25 -62.5) (end 47.788 -54.038) (width 0.75) (layer "B.Cu") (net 10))
 (segment (start 32.307 -57.15) (end 32.307 -59.485) (width 0.635) (layer "B.Cu") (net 10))
 (segment (start 46.5 -89.25) (end 56.25 -79.5) (width 0.75) (layer "B.Cu") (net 10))
 (segment (start 32.307 -57.15) (end 32.307 -54.643) (width 0.635) (layer "B.Cu") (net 10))
 (segment (start 39.034 -54.254) (end 39.25 -54.038) (width 1.016) (layer "B.Cu") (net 10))
 (segment (start 33.588 -54.038) (end 33.25 -53.7) (width 1.016) (layer "B.Cu") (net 10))
 (segment (start 50.75 -73) (end 45.568 -67.818) (width 1.016) (layer "B.Cu") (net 5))
 (segment (start 48.08 -80) (end 48.08 -79.67) (width 1.016) (layer "B.Cu") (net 5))
 (segment (start 48.08 -79.67) (end 50.75 -77) (width 1.016) (layer "B.Cu") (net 5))
 (segment (start 45.568 -67.818) (end 42.926 -67.818) (width 1.016) (layer "B.Cu") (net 5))
 (segment (start 50.75 -77) (end 50.75 -73) (width 1.016) (layer "B.Cu") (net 5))
 (segment (start 37.846 -62.738) (end 37.846 -59.944) (width 1.016) (layer "B.Cu") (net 5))
 (segment (start 42.926 -67.818) (end 37.846 -62.738) (width 1.016) (layer "B.Cu") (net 5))
 (segment (start 32.766 -80.766) (end 36.5 -84.5) (width 0.5) (layer "B.Cu") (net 6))
 (segment (start 45.54 -82.71) (end 45.54 -80) (width 0.5) (layer "B.Cu") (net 6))
 (segment (start 43.75 -84.5) (end 45.54 -82.71) (width 0.5) (layer "B.Cu") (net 6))
 (segment (start 32.766 -76.109) (end 32.766 -80.766) (width 0.5) (layer "B.Cu") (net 6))
 (segment (start 45.54 -79.0015) (end 45.54 -80) (width 0.508) (layer "B.Cu") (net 6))
 (segment (start 36.5 -84.5) (end 43.75 -84.5) (width 0.5) (layer "B.Cu") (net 6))
 (segment (start 43 -82.25) (end 43 -80) (width 0.5) (layer "B.Cu") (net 7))
 (segment (start 37.25 -83) (end 42.25 -83) (width 0.5) (layer "B.Cu") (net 7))
 (segment (start 43 -80) (end 43 -78.92) (width 0.381) (layer "B.Cu") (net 7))
 (segment (start 35.306 -81.056) (end 37.25 -83) (width 0.5) (layer "B.Cu") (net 7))
 (segment (start 35.306 -76.109) (end 35.306 -81.056) (width 0.5) (layer "B.Cu") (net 7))
 (segment (start 35.92525 -75.6465) (end 35.56 -76.01175) (width 0.635) (layer "B.Cu") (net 7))
 (segment (start 42.25 -83) (end 43 -82.25) (width 0.5) (layer "B.Cu") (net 7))
 (segment (start 40.46 -80) (end 40.46 -76.183) (width 0.5) (layer "B.Cu") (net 8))
 (segment (start 40.46 -76.183) (end 40.386 -76.109) (width 1.016) (layer "B.Cu") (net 8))
 (segment (start 45.5 -18) (end 45.5 -20.75) (width 0.75) (layer "B.Cu") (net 3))
 (segment (start 44.5 -24.588) (end 44.45 -24.638) (width 0.75) (layer "B.Cu") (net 3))
 (segment (start 44.5 -21.75) (end 44.5 -24.588) (width 0.75) (layer "B.Cu") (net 3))
 (segment (start 45.5 -15.25) (end 45.5 -18) (width 0.75) (layer "B.Cu") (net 3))
 (segment (start 40.17 -9.92) (end 45.5 -15.25) (width 0.75) (layer "B.Cu") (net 3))
 (segment (start 45.5 -20.75) (end 44.5 -21.75) (width 0.75) (layer "B.Cu") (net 3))
 (segment (start 40.17 -6.75) (end 40.17 -9.92) (width 0.75) (layer "B.Cu") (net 3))
 (segment (start 45.25 -8.75) (end 45.25 -6.75) (width 0.75) (layer "B.Cu") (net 4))
 (segment (start 50.5 -18) (end 50.5 -14) (width 0.75) (layer "B.Cu") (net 4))
 (segment (start 50.5 -23.588) (end 50.5 -18) (width 0.75) (layer "B.Cu") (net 4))
 (segment (start 50.5 -14) (end 45.25 -8.75) (width 0.75) (layer "B.Cu") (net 4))
 (segment (start 49.45 -24.638) (end 50.5 -23.588) (width 0.75) (layer "B.Cu") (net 4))
 (segment (start 43.25 -86) (end 45.5 -86) (width 0.5) (layer "B.Cu") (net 12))
 (segment (start 45.466 -64.466) (end 45.466 -59.944) (width 0.5) (layer "B.Cu") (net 12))
 (segment (start 52.75 -78.75) (end 52.75 -71.75) (width 0.5) (layer "B.Cu") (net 12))
 (segment (start 52.75 -71.75) (end 45.466 -64.466) (width 0.5) (layer "B.Cu") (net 12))
 (segment (start 45.5 -86) (end 52.75 -78.75) (width 0.5) (layer "B.Cu") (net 12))
 (segment (start 41.5 -87.75) (end 43.25 -86) (width 0.5) (layer "B.Cu") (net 12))
 (segment (start 41.5 -90.45) (end 41.5 -87.75) (width 0.5) (layer "B.Cu") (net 12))
 (segment (start 48.006 -76.109) (end 48.006 -76.5355) (width 0.508) (layer "B.Cu") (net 15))
 (segment (start 54.25 -79.25) (end 54.25 -70.25) (width 0.5) (layer "B.Cu") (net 11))
 (segment (start 48.006 -64.006) (end 48.006 -59.944) (width 0.5) (layer "B.Cu") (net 11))
 (segment (start 44.75 -87.5) (end 46 -87.5) (width 0.5) (layer "B.Cu") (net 11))
 (segment (start 44 -90.45) (end 44 -88.25) (width 0.5) (layer "B.Cu") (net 11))
 (segment (start 54.25 -70.25) (end 48.006 -64.006) (width 0.5) (layer "B.Cu") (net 11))
 (segment (start 46 -87.5) (end 54.25 -79.25) (width 0.5) (layer "B.Cu") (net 11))
 (segment (start 44 -88.25) (end 44.75 -87.5) (width 0.5) (layer "B.Cu") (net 11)))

